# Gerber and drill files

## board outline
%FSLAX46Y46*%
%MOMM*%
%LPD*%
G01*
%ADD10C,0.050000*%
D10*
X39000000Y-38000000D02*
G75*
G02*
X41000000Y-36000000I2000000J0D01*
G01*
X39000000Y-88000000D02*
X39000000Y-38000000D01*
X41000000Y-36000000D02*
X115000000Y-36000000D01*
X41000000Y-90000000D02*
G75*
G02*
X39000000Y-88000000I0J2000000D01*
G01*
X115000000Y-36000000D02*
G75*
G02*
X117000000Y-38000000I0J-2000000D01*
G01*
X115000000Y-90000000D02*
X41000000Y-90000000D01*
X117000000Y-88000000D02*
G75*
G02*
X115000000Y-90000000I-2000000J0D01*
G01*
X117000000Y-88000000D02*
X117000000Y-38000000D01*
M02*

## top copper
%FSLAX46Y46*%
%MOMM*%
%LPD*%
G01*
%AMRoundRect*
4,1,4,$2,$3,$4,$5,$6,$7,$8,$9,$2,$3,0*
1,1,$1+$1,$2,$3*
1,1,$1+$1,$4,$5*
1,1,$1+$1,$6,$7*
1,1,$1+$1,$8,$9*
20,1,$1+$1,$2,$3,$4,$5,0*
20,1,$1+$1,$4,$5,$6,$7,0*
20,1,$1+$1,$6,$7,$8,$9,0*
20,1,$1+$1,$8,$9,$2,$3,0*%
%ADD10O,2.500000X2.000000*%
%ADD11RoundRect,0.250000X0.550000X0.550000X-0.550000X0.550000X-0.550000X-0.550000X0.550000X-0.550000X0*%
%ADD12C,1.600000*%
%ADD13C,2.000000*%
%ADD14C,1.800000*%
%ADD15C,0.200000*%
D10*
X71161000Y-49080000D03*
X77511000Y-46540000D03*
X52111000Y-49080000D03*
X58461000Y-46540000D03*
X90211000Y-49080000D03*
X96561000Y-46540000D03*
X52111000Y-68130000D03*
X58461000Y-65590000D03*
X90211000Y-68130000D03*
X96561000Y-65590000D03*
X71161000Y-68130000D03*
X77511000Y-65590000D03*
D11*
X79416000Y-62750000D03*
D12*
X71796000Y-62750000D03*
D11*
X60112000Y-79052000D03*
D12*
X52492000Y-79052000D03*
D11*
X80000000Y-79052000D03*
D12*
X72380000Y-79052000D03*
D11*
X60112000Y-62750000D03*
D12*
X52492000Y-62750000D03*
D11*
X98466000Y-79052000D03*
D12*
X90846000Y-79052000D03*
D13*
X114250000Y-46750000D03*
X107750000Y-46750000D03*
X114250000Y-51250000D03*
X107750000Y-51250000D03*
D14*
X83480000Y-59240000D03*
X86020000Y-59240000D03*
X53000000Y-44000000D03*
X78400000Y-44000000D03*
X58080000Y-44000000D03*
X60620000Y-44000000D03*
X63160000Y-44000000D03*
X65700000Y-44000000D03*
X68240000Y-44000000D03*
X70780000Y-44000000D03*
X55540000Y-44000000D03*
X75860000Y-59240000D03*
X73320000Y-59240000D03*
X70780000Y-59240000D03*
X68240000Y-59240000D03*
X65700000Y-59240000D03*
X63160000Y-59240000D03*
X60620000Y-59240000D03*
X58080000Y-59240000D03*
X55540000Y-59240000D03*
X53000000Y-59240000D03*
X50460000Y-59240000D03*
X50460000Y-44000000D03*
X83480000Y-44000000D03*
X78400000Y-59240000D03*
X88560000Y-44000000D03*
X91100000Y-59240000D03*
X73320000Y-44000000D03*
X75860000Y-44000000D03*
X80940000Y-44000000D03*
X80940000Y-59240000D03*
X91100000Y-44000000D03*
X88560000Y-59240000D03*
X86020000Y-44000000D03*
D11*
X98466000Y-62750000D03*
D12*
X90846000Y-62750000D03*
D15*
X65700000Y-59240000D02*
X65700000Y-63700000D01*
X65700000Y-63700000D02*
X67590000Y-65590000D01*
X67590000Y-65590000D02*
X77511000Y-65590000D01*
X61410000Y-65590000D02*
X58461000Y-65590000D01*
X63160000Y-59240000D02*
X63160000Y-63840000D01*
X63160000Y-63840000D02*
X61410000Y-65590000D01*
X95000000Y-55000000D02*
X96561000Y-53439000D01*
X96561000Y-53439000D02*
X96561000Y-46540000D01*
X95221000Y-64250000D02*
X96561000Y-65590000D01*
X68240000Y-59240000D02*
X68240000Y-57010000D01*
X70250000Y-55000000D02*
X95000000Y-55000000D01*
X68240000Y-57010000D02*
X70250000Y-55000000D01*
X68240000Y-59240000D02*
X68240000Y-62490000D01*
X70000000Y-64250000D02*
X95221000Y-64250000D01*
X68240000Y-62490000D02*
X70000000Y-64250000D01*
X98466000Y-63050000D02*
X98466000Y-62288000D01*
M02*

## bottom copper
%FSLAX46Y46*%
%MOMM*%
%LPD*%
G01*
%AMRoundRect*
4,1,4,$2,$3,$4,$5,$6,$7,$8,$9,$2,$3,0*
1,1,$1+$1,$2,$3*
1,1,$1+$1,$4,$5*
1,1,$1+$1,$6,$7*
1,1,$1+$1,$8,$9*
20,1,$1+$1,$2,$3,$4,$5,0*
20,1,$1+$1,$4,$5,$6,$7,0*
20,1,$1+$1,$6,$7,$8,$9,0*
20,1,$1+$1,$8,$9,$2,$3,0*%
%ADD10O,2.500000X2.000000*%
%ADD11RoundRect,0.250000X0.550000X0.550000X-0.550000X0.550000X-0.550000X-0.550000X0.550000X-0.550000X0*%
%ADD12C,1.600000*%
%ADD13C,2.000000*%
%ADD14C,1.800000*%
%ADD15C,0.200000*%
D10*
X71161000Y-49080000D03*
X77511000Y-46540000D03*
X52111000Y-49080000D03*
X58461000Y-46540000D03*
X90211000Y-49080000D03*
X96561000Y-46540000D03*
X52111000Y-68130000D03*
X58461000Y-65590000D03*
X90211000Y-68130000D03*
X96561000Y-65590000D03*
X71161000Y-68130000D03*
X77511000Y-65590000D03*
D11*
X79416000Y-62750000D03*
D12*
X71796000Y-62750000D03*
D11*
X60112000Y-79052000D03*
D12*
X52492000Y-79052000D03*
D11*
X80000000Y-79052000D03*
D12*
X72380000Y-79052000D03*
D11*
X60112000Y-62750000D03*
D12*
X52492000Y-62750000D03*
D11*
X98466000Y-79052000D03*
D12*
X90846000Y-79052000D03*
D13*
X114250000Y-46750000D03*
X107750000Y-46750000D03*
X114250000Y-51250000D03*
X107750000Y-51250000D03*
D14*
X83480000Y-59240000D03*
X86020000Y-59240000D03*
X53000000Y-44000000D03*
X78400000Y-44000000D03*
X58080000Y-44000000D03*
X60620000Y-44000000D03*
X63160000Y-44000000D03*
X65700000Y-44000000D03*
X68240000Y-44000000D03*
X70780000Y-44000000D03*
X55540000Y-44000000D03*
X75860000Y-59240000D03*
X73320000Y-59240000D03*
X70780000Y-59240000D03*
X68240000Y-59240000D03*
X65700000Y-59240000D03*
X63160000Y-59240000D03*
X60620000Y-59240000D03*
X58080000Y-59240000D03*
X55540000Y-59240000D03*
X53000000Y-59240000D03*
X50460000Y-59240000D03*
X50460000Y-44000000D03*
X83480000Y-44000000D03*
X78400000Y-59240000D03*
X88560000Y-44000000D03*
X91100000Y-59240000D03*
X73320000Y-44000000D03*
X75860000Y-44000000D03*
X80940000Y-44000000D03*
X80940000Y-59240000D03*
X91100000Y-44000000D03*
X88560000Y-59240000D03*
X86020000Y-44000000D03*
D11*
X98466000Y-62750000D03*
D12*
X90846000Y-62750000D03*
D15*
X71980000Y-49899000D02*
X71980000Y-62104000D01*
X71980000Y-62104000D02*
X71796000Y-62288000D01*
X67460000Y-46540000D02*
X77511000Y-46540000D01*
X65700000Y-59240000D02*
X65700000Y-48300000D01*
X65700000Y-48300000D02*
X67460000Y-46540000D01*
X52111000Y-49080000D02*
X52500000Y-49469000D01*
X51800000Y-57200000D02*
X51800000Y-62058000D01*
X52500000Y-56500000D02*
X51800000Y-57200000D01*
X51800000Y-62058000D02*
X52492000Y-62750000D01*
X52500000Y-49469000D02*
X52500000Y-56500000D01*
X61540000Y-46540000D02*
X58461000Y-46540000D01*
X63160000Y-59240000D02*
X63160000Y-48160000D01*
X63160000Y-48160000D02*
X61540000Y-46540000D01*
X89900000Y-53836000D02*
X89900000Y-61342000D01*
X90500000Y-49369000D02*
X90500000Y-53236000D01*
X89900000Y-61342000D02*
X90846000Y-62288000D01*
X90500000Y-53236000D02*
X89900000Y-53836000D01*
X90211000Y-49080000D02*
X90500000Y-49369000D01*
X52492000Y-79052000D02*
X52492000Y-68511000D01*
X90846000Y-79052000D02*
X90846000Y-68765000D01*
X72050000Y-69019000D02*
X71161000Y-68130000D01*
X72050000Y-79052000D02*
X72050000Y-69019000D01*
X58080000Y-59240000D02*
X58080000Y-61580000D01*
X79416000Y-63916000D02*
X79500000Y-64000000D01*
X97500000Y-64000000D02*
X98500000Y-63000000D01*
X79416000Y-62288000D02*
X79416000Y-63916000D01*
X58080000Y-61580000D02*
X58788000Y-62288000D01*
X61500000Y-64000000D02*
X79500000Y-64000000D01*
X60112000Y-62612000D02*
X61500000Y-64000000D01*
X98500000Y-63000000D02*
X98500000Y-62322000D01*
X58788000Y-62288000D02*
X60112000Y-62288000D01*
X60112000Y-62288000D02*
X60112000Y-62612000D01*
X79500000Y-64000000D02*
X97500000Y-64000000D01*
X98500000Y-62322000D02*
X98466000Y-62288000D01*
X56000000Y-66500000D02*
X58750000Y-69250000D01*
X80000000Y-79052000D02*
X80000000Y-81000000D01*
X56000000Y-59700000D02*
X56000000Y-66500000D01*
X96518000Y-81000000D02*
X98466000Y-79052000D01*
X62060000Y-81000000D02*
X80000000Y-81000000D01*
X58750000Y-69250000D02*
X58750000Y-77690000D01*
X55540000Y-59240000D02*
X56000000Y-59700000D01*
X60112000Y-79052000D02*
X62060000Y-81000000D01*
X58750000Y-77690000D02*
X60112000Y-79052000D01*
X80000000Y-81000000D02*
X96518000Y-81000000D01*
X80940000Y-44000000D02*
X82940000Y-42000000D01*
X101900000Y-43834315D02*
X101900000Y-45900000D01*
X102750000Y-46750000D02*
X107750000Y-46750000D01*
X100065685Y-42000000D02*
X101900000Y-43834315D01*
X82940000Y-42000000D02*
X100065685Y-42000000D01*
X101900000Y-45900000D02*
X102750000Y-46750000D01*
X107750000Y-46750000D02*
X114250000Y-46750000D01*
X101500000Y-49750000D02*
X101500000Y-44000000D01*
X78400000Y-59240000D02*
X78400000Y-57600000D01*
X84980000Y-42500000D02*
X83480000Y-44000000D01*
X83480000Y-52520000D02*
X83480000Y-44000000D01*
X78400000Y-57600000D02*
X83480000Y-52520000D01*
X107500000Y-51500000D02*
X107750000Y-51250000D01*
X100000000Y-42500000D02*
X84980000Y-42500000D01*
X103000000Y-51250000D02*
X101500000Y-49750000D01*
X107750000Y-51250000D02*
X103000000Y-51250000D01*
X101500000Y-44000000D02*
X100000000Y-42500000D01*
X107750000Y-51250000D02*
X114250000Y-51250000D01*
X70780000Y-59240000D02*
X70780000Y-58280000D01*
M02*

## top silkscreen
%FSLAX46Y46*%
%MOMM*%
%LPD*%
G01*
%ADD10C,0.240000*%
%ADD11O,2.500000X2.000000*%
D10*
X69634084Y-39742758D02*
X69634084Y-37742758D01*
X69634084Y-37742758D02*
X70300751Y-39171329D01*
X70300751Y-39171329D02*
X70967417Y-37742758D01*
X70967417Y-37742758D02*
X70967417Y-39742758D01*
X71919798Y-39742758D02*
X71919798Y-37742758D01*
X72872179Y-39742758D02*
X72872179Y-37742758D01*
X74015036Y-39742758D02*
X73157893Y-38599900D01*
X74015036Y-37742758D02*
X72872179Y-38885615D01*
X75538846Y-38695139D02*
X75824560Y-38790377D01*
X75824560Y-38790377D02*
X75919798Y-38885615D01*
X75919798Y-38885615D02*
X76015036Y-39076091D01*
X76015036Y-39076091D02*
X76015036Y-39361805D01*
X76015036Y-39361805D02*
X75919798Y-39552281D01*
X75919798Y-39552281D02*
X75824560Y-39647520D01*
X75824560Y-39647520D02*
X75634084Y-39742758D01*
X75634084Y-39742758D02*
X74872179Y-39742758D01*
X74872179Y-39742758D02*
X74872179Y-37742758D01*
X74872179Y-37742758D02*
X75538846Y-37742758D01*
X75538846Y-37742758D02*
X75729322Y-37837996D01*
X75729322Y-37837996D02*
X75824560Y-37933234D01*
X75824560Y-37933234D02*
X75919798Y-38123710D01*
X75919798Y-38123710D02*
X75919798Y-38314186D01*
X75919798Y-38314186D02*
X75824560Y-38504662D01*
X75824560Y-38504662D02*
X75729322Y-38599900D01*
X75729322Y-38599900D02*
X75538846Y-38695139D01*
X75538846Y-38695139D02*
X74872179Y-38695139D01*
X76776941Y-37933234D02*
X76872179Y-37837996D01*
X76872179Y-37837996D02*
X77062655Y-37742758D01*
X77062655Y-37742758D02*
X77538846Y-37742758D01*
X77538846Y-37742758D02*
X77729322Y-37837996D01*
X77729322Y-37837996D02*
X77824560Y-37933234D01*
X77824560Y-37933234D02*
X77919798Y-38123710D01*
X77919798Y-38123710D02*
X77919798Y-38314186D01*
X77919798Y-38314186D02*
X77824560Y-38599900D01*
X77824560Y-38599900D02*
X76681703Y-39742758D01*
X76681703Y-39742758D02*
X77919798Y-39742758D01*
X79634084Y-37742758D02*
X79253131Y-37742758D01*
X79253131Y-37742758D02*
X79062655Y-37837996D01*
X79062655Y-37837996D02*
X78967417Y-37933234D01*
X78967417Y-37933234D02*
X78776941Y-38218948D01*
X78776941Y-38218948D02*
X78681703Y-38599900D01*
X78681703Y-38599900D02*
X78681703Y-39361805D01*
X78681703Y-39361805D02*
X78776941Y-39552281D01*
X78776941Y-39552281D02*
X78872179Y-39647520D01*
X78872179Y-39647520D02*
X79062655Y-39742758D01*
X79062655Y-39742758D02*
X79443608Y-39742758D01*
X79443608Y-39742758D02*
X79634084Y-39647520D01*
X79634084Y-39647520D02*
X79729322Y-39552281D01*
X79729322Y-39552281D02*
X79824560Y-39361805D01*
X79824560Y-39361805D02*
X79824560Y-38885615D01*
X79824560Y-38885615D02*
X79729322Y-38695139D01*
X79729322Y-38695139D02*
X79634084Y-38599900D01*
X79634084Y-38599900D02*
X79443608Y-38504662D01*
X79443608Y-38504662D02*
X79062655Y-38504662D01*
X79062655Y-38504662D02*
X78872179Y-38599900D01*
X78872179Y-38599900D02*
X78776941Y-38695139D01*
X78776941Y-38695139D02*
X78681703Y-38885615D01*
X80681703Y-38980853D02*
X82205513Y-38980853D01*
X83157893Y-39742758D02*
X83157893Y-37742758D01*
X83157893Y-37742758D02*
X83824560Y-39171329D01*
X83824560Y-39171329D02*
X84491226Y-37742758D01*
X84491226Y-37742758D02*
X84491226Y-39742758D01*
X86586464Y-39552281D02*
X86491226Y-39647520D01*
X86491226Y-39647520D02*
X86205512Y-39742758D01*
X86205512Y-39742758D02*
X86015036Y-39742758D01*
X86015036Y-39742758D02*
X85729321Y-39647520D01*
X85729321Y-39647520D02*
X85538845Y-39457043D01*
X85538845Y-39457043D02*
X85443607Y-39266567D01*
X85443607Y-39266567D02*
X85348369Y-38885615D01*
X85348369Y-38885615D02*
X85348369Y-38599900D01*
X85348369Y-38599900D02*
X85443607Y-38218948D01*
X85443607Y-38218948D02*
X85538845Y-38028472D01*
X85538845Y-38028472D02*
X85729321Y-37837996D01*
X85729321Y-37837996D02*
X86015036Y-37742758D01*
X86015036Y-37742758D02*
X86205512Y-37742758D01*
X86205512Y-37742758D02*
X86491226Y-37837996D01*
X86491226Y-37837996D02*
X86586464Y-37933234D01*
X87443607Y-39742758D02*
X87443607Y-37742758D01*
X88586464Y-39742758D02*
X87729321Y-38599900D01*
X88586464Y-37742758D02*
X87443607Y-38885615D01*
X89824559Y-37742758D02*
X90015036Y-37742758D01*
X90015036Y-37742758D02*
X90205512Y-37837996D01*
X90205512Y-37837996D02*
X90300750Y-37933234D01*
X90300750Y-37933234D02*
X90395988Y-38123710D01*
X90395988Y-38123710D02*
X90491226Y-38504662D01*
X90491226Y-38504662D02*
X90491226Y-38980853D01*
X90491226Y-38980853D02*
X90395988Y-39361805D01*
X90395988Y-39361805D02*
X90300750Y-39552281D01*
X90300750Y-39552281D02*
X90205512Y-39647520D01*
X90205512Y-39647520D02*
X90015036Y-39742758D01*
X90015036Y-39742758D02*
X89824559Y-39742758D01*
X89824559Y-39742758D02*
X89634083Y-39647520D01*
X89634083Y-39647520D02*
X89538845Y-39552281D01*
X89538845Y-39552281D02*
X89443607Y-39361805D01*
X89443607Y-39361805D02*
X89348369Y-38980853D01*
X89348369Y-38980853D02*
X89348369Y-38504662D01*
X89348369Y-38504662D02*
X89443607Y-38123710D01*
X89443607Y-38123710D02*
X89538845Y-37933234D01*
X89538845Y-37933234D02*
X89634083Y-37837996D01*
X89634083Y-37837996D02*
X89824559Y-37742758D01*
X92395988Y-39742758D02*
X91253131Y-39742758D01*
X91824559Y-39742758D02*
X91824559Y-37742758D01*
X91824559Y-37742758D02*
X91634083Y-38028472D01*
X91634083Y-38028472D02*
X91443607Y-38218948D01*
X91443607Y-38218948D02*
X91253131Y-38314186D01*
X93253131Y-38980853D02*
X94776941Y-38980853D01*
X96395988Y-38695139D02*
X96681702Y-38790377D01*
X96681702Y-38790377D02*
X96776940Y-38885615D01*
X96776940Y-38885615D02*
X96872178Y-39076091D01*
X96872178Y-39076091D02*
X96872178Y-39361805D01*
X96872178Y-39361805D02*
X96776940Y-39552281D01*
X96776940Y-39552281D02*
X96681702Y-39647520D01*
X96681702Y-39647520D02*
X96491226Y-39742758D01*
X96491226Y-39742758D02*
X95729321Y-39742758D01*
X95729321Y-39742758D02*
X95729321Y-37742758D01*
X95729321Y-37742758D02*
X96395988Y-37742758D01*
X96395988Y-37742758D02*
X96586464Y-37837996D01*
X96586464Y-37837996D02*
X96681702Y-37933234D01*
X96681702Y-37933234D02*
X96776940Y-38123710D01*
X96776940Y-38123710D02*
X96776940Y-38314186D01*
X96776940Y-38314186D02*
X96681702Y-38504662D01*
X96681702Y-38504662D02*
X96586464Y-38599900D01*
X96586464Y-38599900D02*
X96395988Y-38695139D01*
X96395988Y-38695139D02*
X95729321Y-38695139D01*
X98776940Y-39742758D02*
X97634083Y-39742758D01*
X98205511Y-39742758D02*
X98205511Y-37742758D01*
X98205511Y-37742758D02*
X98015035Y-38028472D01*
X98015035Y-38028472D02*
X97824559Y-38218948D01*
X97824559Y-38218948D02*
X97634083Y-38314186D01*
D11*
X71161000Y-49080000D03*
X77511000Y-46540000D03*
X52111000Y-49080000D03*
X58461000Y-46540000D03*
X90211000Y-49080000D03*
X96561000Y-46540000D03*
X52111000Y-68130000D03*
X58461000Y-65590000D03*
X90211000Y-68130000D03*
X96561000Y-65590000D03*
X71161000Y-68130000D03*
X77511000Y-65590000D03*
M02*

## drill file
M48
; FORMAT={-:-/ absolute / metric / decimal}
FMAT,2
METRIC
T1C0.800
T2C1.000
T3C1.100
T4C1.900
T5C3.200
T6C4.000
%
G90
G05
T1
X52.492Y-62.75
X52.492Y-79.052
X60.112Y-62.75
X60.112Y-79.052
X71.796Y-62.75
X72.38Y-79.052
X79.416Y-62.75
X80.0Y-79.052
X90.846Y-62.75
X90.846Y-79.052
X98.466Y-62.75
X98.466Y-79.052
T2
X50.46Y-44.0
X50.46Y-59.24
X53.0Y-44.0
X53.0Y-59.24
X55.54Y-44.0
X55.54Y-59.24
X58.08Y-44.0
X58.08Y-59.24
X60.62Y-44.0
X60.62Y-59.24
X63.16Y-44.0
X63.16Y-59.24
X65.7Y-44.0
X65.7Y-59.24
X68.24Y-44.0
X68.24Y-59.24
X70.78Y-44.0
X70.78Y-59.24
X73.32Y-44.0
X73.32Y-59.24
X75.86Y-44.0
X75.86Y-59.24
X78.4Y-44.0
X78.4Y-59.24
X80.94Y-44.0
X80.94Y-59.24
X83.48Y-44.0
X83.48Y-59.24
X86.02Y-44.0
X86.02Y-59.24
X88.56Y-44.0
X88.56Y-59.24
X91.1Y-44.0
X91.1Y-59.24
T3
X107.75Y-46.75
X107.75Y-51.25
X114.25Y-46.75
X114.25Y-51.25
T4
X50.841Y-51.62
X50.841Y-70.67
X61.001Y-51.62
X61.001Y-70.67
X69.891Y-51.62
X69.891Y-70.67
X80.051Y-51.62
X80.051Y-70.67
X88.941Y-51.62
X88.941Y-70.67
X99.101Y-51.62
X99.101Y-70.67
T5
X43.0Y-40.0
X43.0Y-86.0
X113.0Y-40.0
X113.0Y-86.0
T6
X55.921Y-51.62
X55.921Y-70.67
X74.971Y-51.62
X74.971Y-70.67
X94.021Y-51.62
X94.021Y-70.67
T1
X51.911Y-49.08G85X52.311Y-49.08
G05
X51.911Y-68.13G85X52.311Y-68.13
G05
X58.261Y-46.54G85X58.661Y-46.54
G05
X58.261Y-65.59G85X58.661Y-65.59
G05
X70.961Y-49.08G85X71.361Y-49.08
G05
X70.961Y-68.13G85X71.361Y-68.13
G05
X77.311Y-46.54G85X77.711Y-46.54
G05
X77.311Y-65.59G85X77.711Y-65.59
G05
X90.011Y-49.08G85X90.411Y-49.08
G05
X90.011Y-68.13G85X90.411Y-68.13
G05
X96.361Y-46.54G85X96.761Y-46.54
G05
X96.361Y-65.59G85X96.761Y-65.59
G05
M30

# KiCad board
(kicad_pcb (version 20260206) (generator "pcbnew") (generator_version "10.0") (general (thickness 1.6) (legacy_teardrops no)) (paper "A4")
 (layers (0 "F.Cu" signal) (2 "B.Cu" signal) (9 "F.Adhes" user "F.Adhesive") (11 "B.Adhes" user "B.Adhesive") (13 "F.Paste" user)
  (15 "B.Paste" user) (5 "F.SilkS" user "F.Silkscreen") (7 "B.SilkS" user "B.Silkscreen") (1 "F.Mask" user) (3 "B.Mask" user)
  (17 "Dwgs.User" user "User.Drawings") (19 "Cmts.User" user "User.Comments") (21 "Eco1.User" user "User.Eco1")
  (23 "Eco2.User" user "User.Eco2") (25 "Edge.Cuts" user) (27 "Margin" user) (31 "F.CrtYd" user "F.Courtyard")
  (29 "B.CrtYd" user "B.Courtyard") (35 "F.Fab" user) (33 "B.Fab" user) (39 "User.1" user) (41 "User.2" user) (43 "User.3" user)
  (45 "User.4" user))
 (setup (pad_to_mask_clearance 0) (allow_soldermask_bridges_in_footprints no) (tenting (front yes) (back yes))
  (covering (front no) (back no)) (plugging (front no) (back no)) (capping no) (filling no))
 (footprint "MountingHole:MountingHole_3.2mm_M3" (layer "F.Cu") (at 113 40 180)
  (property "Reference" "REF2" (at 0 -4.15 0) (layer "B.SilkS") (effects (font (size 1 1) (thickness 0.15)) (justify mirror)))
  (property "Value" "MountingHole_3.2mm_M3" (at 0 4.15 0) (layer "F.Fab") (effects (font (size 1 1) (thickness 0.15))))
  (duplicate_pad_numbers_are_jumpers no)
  (pad "" np_thru_hole circle (at 0 0 180) (size 3.2 3.2) (drill 3.2) (layers "*.Cu" "*.Mask")))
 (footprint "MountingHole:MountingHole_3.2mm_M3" (layer "F.Cu") (at 113 86)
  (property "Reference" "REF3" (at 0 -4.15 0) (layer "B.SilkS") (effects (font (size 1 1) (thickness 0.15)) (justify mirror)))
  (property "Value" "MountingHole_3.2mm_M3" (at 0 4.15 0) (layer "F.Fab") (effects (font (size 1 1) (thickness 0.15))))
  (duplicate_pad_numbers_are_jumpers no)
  (pad "" np_thru_hole circle (at 0 0) (size 3.2 3.2) (drill 3.2) (layers "*.Cu" "*.Mask")))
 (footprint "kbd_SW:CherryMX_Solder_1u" (layer "F.Cu") (at 74.971 51.62)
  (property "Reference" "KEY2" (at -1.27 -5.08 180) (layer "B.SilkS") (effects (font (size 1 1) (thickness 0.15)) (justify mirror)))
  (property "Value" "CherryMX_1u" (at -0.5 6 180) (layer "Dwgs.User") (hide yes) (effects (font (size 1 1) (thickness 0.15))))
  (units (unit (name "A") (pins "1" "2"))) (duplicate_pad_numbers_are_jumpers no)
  (pad "" np_thru_hole circle (at -5.08 0 90) (size 1.9 1.9) (drill 1.9) (layers "*.Cu" "*.Mask"))
  (pad "" np_thru_hole circle (at 0 0 90) (size 4 4) (drill 4) (layers "*.Cu" "*.Mask"))
  (pad "" np_thru_hole circle (at 5.08 0 90) (size 1.9 1.9) (drill 1.9) (layers "*.Cu" "*.Mask"))
  (pad "1" thru_hole oval (at -3.81 -2.54) (size 2.5 2) (drill oval 1.2 0.8) (layers "*.Cu" "B.Mask" "F.SilkS") (remove_unused_layers no)
   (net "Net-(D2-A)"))
  (pad "2" thru_hole oval (at 2.54 -5.08) (size 2.5 2) (drill oval 1.2 0.8) (layers "*.Cu" "B.Mask" "F.SilkS") (remove_unused_layers no)
   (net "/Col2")))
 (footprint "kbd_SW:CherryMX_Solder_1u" (layer "F.Cu") (at 55.921 51.62)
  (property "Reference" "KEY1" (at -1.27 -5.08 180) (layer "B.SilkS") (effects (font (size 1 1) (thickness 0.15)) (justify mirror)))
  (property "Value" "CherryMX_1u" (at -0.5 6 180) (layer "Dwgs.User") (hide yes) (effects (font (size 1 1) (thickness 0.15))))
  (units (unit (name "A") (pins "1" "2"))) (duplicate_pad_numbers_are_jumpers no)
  (pad "" np_thru_hole circle (at -5.08 0 90) (size 1.9 1.9) (drill 1.9) (layers "*.Cu" "*.Mask"))
  (pad "" np_thru_hole circle (at 0 0 90) (size 4 4) (drill 4) (layers "*.Cu" "*.Mask"))
  (pad "" np_thru_hole circle (at 5.08 0 90) (size 1.9 1.9) (drill 1.9) (layers "*.Cu" "*.Mask"))
  (pad "1" thru_hole oval (at -3.81 -2.54) (size 2.5 2) (drill oval 1.2 0.8) (layers "*.Cu" "B.Mask" "F.SilkS") (remove_unused_layers no)
   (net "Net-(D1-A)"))
  (pad "2" thru_hole oval (at 2.54 -5.08) (size 2.5 2) (drill oval 1.2 0.8) (layers "*.Cu" "B.Mask" "F.SilkS") (remove_unused_layers no)
   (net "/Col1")))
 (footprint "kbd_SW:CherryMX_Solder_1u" (layer "F.Cu") (at 94.021 51.62)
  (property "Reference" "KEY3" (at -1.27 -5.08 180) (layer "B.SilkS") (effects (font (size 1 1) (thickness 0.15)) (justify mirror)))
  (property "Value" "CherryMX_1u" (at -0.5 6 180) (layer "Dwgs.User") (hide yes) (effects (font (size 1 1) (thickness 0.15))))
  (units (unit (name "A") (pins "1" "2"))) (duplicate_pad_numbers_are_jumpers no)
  (pad "" np_thru_hole circle (at -5.08 0 90) (size 1.9 1.9) (drill 1.9) (layers "*.Cu" "*.Mask"))
  (pad "" np_thru_hole circle (at 0 0 90) (size 4 4) (drill 4) (layers "*.Cu" "*.Mask"))
  (pad "" np_thru_hole circle (at 5.08 0 90) (size 1.9 1.9) (drill 1.9) (layers "*.Cu" "*.Mask"))
  (pad "1" thru_hole oval (at -3.81 -2.54) (size 2.5 2) (drill oval 1.2 0.8) (layers "*.Cu" "B.Mask" "F.SilkS") (remove_unused_layers no)
   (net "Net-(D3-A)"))
  (pad "2" thru_hole oval (at 2.54 -5.08) (size 2.5 2) (drill oval 1.2 0.8) (layers "*.Cu" "B.Mask" "F.SilkS") (remove_unused_layers no)
   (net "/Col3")))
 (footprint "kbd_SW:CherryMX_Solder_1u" (layer "F.Cu") (at 55.921 70.67)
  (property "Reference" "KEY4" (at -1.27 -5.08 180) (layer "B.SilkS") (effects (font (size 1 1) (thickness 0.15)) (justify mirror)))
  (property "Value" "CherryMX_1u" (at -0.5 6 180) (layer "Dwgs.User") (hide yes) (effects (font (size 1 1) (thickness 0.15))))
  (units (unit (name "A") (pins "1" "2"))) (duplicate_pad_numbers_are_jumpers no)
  (pad "" np_thru_hole circle (at -5.08 0 90) (size 1.9 1.9) (drill 1.9) (layers "*.Cu" "*.Mask"))
  (pad "" np_thru_hole circle (at 0 0 90) (size 4 4) (drill 4) (layers "*.Cu" "*.Mask"))
  (pad "" np_thru_hole circle (at 5.08 0 90) (size 1.9 1.9) (drill 1.9) (layers "*.Cu" "*.Mask"))
  (pad "1" thru_hole oval (at -3.81 -2.54) (size 2.5 2) (drill oval 1.2 0.8) (layers "*.Cu" "B.Mask" "F.SilkS") (remove_unused_layers no)
   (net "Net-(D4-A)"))
  (pad "2" thru_hole oval (at 2.54 -5.08) (size 2.5 2) (drill oval 1.2 0.8) (layers "*.Cu" "B.Mask" "F.SilkS") (remove_unused_layers no)
   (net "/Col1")))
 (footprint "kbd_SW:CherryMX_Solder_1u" (layer "F.Cu") (at 94.021 70.67)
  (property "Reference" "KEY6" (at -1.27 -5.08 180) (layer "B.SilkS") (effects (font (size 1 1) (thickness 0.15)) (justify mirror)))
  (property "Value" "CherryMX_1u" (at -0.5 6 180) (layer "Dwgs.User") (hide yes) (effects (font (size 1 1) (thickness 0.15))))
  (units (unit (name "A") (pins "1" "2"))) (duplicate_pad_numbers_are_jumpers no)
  (pad "" np_thru_hole circle (at -5.08 0 90) (size 1.9 1.9) (drill 1.9) (layers "*.Cu" "*.Mask"))
  (pad "" np_thru_hole circle (at 0 0 90) (size 4 4) (drill 4) (layers "*.Cu" "*.Mask"))
  (pad "" np_thru_hole circle (at 5.08 0 90) (size 1.9 1.9) (drill 1.9) (layers "*.Cu" "*.Mask"))
  (pad "1" thru_hole oval (at -3.81 -2.54) (size 2.5 2) (drill oval 1.2 0.8) (layers "*.Cu" "B.Mask" "F.SilkS") (remove_unused_layers no)
   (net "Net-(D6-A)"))
  (pad "2" thru_hole oval (at 2.54 -5.08) (size 2.5 2) (drill oval 1.2 0.8) (layers "*.Cu" "B.Mask" "F.SilkS") (remove_unused_layers no)
   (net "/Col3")))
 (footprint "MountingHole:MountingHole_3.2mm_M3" (layer "F.Cu") (at 43 40 180)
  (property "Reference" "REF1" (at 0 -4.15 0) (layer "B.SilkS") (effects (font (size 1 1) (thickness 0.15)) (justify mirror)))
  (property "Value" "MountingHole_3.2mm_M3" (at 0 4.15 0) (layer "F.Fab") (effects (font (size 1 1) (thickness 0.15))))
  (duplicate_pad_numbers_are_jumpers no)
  (pad "" np_thru_hole circle (at 0 0 180) (size 3.2 3.2) (drill 3.2) (layers "*.Cu" "*.Mask")))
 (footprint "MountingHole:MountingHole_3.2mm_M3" (layer "F.Cu") (at 43 86)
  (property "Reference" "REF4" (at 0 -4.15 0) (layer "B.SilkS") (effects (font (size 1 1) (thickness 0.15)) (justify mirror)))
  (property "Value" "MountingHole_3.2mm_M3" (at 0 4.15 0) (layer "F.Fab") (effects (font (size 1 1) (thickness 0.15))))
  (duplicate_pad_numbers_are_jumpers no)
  (pad "" np_thru_hole circle (at 0 0) (size 3.2 3.2) (drill 3.2) (layers "*.Cu" "*.Mask")))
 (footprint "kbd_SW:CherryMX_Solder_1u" (layer "F.Cu") (at 74.971 70.67)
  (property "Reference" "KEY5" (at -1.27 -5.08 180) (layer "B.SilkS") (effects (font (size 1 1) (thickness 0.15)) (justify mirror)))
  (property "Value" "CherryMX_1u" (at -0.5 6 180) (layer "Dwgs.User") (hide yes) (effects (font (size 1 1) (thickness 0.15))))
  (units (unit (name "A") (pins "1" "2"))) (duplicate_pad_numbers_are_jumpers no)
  (pad "" np_thru_hole circle (at -5.08 0 90) (size 1.9 1.9) (drill 1.9) (layers "*.Cu" "*.Mask"))
  (pad "" np_thru_hole circle (at 0 0 90) (size 4 4) (drill 4) (layers "*.Cu" "*.Mask"))
  (pad "" np_thru_hole circle (at 5.08 0 90) (size 1.9 1.9) (drill 1.9) (layers "*.Cu" "*.Mask"))
  (pad "1" thru_hole oval (at -3.81 -2.54) (size 2.5 2) (drill oval 1.2 0.8) (layers "*.Cu" "B.Mask" "F.SilkS") (remove_unused_layers no)
   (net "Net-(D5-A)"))
  (pad "2" thru_hole oval (at 2.54 -5.08) (size 2.5 2) (drill oval 1.2 0.8) (layers "*.Cu" "B.Mask" "F.SilkS") (remove_unused_layers no)
   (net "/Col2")))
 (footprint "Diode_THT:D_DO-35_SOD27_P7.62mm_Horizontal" (layer "B.Cu") (at 79.416 62.75 180)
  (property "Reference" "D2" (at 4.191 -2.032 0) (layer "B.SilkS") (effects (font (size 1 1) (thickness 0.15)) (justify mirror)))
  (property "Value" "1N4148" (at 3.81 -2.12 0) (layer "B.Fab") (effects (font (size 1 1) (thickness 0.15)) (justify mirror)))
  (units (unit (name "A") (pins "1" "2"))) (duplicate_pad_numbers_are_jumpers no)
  (pad "1" thru_hole roundrect (at 0 0 180) (size 1.6 1.6) (drill 0.8) (layers "*.Cu" "*.Mask") (remove_unused_layers no)
   (roundrect_rratio 0.15625) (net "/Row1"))
  (pad "2" thru_hole circle (at 7.62 0 180) (size 1.6 1.6) (drill 0.8) (layers "*.Cu" "*.Mask") (remove_unused_layers no) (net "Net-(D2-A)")))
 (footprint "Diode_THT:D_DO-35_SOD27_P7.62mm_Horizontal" (layer "B.Cu") (at 60.112 79.052 180)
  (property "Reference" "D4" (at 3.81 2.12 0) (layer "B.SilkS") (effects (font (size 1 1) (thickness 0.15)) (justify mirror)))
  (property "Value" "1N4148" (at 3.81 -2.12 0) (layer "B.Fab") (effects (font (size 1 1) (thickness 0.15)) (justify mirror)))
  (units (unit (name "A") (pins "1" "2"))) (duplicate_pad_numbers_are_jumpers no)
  (pad "1" thru_hole roundrect (at 0 0 180) (size 1.6 1.6) (drill 0.8) (layers "*.Cu" "*.Mask") (remove_unused_layers no)
   (roundrect_rratio 0.15625) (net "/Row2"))
  (pad "2" thru_hole circle (at 7.62 0 180) (size 1.6 1.6) (drill 0.8) (layers "*.Cu" "*.Mask") (remove_unused_layers no) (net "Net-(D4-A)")))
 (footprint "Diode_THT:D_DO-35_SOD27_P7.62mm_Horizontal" (layer "B.Cu") (at 80 79.052 180)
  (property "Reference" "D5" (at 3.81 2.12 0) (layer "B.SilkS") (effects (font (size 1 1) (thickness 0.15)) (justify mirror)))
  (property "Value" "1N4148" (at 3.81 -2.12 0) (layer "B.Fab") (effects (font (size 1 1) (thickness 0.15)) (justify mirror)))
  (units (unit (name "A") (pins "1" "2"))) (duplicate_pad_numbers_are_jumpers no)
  (pad "1" thru_hole roundrect (at 0 0 180) (size 1.6 1.6) (drill 0.8) (layers "*.Cu" "*.Mask") (remove_unused_layers no)
   (roundrect_rratio 0.15625) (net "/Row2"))
  (pad "2" thru_hole circle (at 7.62 0 180) (size 1.6 1.6) (drill 0.8) (layers "*.Cu" "*.Mask") (remove_unused_layers no) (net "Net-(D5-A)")))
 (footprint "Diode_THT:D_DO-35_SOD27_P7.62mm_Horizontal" (layer "B.Cu") (at 60.112 62.75 180)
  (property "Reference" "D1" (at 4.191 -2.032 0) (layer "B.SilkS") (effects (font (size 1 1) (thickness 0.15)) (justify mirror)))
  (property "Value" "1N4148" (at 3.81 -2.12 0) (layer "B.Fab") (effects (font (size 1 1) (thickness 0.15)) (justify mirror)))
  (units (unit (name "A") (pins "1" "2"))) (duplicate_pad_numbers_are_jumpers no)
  (pad "1" thru_hole roundrect (at 0 0 180) (size 1.6 1.6) (drill 0.8) (layers "*.Cu" "*.Mask") (remove_unused_layers no)
   (roundrect_rratio 0.15625) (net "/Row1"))
  (pad "2" thru_hole circle (at 7.62 0 180) (size 1.6 1.6) (drill 0.8) (layers "*.Cu" "*.Mask") (remove_unused_layers no) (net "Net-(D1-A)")))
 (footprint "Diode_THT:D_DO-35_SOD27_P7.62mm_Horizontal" (layer "B.Cu") (at 98.466 79.052 180)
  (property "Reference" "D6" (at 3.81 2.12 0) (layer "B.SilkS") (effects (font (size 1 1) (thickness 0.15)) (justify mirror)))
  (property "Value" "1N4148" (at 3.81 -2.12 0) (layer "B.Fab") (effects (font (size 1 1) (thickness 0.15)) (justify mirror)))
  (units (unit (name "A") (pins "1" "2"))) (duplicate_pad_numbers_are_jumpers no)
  (pad "1" thru_hole roundrect (at 0 0 180) (size 1.6 1.6) (drill 0.8) (layers "*.Cu" "*.Mask") (remove_unused_layers no)
   (roundrect_rratio 0.15625) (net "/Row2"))
  (pad "2" thru_hole circle (at 7.62 0 180) (size 1.6 1.6) (drill 0.8) (layers "*.Cu" "*.Mask") (remove_unused_layers no) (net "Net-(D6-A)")))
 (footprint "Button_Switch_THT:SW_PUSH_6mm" (layer "B.Cu") (at 114.25 46.75 180)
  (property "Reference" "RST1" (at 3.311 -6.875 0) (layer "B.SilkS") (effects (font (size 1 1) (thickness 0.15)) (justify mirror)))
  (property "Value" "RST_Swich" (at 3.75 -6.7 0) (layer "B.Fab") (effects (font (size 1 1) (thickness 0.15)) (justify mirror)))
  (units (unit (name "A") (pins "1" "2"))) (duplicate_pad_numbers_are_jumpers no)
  (pad "1" thru_hole circle (at 0 0 90) (size 2 2) (drill 1.1) (layers "*.Cu" "*.Mask") (remove_unused_layers no) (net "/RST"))
  (pad "1" thru_hole circle (at 6.5 0 90) (size 2 2) (drill 1.1) (layers "*.Cu" "*.Mask") (remove_unused_layers no) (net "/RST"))
  (pad "2" thru_hole circle (at 0 -4.5 90) (size 2 2) (drill 1.1) (layers "*.Cu" "*.Mask") (remove_unused_layers no) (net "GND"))
  (pad "2" thru_hole circle (at 6.5 -4.5 90) (size 2 2) (drill 1.1) (layers "*.Cu" "*.Mask") (remove_unused_layers no) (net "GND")))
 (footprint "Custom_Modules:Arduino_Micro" (layer "B.Cu") (at 50.46 51.62 -90)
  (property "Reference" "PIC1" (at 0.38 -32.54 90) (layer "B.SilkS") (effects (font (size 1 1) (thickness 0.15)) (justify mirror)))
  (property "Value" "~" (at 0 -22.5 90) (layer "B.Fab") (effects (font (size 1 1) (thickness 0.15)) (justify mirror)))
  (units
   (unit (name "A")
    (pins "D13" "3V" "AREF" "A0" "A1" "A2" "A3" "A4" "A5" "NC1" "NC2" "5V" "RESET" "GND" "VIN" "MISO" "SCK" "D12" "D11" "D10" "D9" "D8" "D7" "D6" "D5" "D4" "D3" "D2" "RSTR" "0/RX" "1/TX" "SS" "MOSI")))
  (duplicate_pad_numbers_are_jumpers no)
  (pad "0/RX" thru_hole circle (at 7.62 -33.02 270) (size 1.8 1.8) (drill 1) (layers "*.Cu" "*.Mask") (remove_unused_layers no)
   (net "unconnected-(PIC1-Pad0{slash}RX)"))
  (pad "1/TX" thru_hole circle (at 7.62 -35.56 270) (size 1.8 1.8) (drill 1) (layers "*.Cu" "*.Mask") (remove_unused_layers no)
   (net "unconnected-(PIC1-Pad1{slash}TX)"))
  (pad "3V" thru_hole circle (at -7.62 -2.54 270) (size 1.8 1.8) (drill 1) (layers "*.Cu" "*.Mask") (remove_unused_layers no)
   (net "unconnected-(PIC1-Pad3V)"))
  (pad "5V" thru_hole circle (at -7.62 -27.94 270) (size 1.8 1.8) (drill 1) (layers "*.Cu" "*.Mask") (remove_unused_layers no)
   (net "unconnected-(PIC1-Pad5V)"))
  (pad "A0" thru_hole circle (at -7.62 -7.62 270) (size 1.8 1.8) (drill 1) (layers "*.Cu" "*.Mask") (remove_unused_layers no)
   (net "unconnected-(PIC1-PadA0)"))
  (pad "A1" thru_hole circle (at -7.62 -10.16 270) (size 1.8 1.8) (drill 1) (layers "*.Cu" "*.Mask") (remove_unused_layers no)
   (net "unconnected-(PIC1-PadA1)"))
  (pad "A2" thru_hole circle (at -7.62 -12.7 270) (size 1.8 1.8) (drill 1) (layers "*.Cu" "*.Mask") (remove_unused_layers no)
   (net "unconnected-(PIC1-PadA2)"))
  (pad "A3" thru_hole circle (at -7.62 -15.24 270) (size 1.8 1.8) (drill 1) (layers "*.Cu" "*.Mask") (remove_unused_layers no)
   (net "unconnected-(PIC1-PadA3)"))
  (pad "A4" thru_hole circle (at -7.62 -17.78 270) (size 1.8 1.8) (drill 1) (layers "*.Cu" "*.Mask") (remove_unused_layers no)
   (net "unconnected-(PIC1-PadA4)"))
  (pad "A5" thru_hole circle (at -7.62 -20.32 270) (size 1.8 1.8) (drill 1) (layers "*.Cu" "*.Mask") (remove_unused_layers no)
   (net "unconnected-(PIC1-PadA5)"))
  (pad "AREF" thru_hole circle (at -7.62 -5.08 270) (size 1.8 1.8) (drill 1) (layers "*.Cu" "*.Mask") (remove_unused_layers no)
   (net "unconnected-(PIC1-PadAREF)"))
  (pad "D2" thru_hole circle (at 7.62 -25.4 270) (size 1.8 1.8) (drill 1) (layers "*.Cu" "*.Mask") (remove_unused_layers no)
   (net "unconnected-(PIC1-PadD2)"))
  (pad "D3" thru_hole circle (at 7.62 -22.86 270) (size 1.8 1.8) (drill 1) (layers "*.Cu" "*.Mask") (remove_unused_layers no)
   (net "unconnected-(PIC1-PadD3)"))
  (pad "D4" thru_hole circle (at 7.62 -20.32 270) (size 1.8 1.8) (drill 1) (layers "*.Cu" "*.Mask") (remove_unused_layers no)
   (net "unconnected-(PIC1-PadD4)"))
  (pad "D5" thru_hole circle (at 7.62 -17.78 270) (size 1.8 1.8) (drill 1) (layers "*.Cu" "*.Mask") (remove_unused_layers no) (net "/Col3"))
  (pad "D6" thru_hole circle (at 7.62 -15.24 270) (size 1.8 1.8) (drill 1) (layers "*.Cu" "*.Mask") (remove_unused_layers no) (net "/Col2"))
  (pad "D7" thru_hole circle (at 7.62 -12.7 270) (size 1.8 1.8) (drill 1) (layers "*.Cu" "*.Mask") (remove_unused_layers no) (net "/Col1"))
  (pad "D8" thru_hole circle (at 7.62 -10.16 270) (size 1.8 1.8) (drill 1) (layers "*.Cu" "*.Mask") (remove_unused_layers no)
   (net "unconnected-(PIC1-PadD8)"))
  (pad "D9" thru_hole circle (at 7.62 -7.62 270) (size 1.8 1.8) (drill 1) (layers "*.Cu" "*.Mask") (remove_unused_layers no) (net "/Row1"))
  (pad "D10" thru_hole circle (at 7.62 -5.08 270) (size 1.8 1.8) (drill 1) (layers "*.Cu" "*.Mask") (remove_unused_layers no) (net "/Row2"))
  (pad "D11" thru_hole circle (at 7.62 -2.54 270) (size 1.8 1.8) (drill 1) (layers "*.Cu" "*.Mask") (remove_unused_layers no)
   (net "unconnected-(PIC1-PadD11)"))
  (pad "D12" thru_hole circle (at 7.62 0 270) (size 1.8 1.8) (drill 1) (layers "*.Cu" "*.Mask") (remove_unused_layers no)
   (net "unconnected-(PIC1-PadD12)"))
  (pad "D13" thru_hole circle (at -7.62 0 270) (size 1.8 1.8) (drill 1) (layers "*.Cu" "*.Mask") (remove_unused_layers no)
   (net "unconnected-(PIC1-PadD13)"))
  (pad "GND" thru_hole circle (at -7.62 -33.02 270) (size 1.8 1.8) (drill 1) (layers "*.Cu" "*.Mask") (remove_unused_layers no) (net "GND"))
  (pad "GND" thru_hole circle (at 7.62 -27.94 270) (size 1.8 1.8) (drill 1) (layers "*.Cu" "*.Mask") (remove_unused_layers no) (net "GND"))
  (pad "MISO" thru_hole circle (at -7.62 -38.1 270) (size 1.8 1.8) (drill 1) (layers "*.Cu" "*.Mask") (remove_unused_layers no)
   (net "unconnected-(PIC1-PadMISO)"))
  (pad "MOSI" thru_hole circle (at 7.62 -40.64 270) (size 1.8 1.8) (drill 1) (layers "*.Cu" "*.Mask") (remove_unused_layers no)
   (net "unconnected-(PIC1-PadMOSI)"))
  (pad "NC1" thru_hole circle (at -7.62 -22.86 270) (size 1.8 1.8) (drill 1) (layers "*.Cu" "*.Mask") (remove_unused_layers no)
   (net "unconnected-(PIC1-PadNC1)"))
  (pad "NC2" thru_hole circle (at -7.62 -25.4 270) (size 1.8 1.8) (drill 1) (layers "*.Cu" "*.Mask") (remove_unused_layers no)
   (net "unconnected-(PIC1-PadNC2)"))
  (pad "RESET" thru_hole circle (at -7.62 -30.48 270) (size 1.8 1.8) (drill 1) (layers "*.Cu" "*.Mask") (remove_unused_layers no)
   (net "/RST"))
  (pad "RSTR" thru_hole circle (at 7.62 -30.48 270) (size 1.8 1.8) (drill 1) (layers "*.Cu" "*.Mask") (remove_unused_layers no)
   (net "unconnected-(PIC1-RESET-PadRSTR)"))
  (pad "SCK" thru_hole circle (at -7.62 -40.64 270) (size 1.8 1.8) (drill 1) (layers "*.Cu" "*.Mask") (remove_unused_layers no)
   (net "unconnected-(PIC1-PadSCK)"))
  (pad "SS" thru_hole circle (at 7.62 -38.1 270) (size 1.8 1.8) (drill 1) (layers "*.Cu" "*.Mask") (remove_unused_layers no)
   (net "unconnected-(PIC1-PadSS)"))
  (pad "VIN" thru_hole circle (at -7.62 -35.56 270) (size 1.8 1.8) (drill 1) (layers "*.Cu" "*.Mask") (remove_unused_layers no)
   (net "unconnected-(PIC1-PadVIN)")))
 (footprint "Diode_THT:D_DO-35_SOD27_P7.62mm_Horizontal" (layer "B.Cu") (at 98.466 62.75 180)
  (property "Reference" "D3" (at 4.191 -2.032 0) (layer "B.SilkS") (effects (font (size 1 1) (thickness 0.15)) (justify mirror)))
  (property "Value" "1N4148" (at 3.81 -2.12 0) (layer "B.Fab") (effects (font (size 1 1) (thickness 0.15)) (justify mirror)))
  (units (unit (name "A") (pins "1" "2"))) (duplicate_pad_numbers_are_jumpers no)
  (pad "1" thru_hole roundrect (at 0 0 180) (size 1.6 1.6) (drill 0.8) (layers "*.Cu" "*.Mask") (remove_unused_layers no)
   (roundrect_rratio 0.15625) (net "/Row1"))
  (pad "2" thru_hole circle (at 7.62 0 180) (size 1.6 1.6) (drill 0.8) (layers "*.Cu" "*.Mask") (remove_unused_layers no) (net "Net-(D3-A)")))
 (gr_arc (start 39 38) (mid 39.585786 36.585786) (end 41 36) (stroke (width 0.05) (type default)) (layer "Edge.Cuts"))
 (gr_line (start 39 88) (end 39 38) (stroke (width 0.05) (type default)) (layer "Edge.Cuts"))
 (gr_line (start 41 36) (end 115 36) (stroke (width 0.05) (type default)) (layer "Edge.Cuts"))
 (gr_arc (start 41 90) (mid 39.585786 89.414214) (end 39 88) (stroke (width 0.05) (type default)) (layer "Edge.Cuts"))
 (gr_arc (start 115 36) (mid 116.414214 36.585786) (end 117 38) (stroke (width 0.05) (type default)) (layer "Edge.Cuts"))
 (gr_line (start 115 90) (end 41 90) (stroke (width 0.05) (type default)) (layer "Edge.Cuts"))
 (gr_arc (start 117 88) (mid 116.414214 89.414214) (end 115 90) (stroke (width 0.05) (type default)) (layer "Edge.Cuts"))
 (gr_line (start 117 88) (end 117 38) (stroke (width 0.05) (type default)) (layer "Edge.Cuts"))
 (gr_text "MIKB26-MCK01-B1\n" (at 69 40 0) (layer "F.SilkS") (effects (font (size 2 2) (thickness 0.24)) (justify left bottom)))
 (segment (start 71.98 49.899) (end 71.98 62.104) (width 0.2) (layer "B.Cu") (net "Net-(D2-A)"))
 (segment (start 71.98 62.104) (end 71.796 62.288) (width 0.2) (layer "B.Cu") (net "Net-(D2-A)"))
 (segment (start 65.7 59.24) (end 65.7 63.7) (width 0.2) (layer "F.Cu") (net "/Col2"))
 (segment (start 65.7 63.7) (end 67.59 65.59) (width 0.2) (layer "F.Cu") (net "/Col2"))
 (segment (start 67.59 65.59) (end 77.511 65.59) (width 0.2) (layer "F.Cu") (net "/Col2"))
 (segment (start 67.46 46.54) (end 77.511 46.54) (width 0.2) (layer "B.Cu") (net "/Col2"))
 (segment (start 65.7 59.24) (end 65.7 48.3) (width 0.2) (layer "B.Cu") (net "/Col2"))
 (segment (start 65.7 48.3) (end 67.46 46.54) (width 0.2) (layer "B.Cu") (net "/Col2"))
 (segment (start 52.111 49.08) (end 52.5 49.469) (width 0.2) (layer "B.Cu") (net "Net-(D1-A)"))
 (segment (start 51.8 57.2) (end 51.8 62.058) (width 0.2) (layer "B.Cu") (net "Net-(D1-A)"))
 (segment (start 52.5 56.5) (end 51.8 57.2) (width 0.2) (layer "B.Cu") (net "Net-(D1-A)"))
 (segment (start 51.8 62.058) (end 52.492 62.75) (width 0.2) (layer "B.Cu") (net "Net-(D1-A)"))
 (segment (start 52.5 49.469) (end 52.5 56.5) (width 0.2) (layer "B.Cu") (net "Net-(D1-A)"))
 (segment (start 61.41 65.59) (end 58.461 65.59) (width 0.2) (layer "F.Cu") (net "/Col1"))
 (segment (start 63.16 59.24) (end 63.16 63.84) (width 0.2) (layer "F.Cu") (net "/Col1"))
 (segment (start 63.16 63.84) (end 61.41 65.59) (width 0.2) (layer "F.Cu") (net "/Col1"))
 (segment (start 61.54 46.54) (end 58.461 46.54) (width 0.2) (layer "B.Cu") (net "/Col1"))
 (segment (start 63.16 59.24) (end 63.16 48.16) (width 0.2) (layer "B.Cu") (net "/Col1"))
 (segment (start 63.16 48.16) (end 61.54 46.54) (width 0.2) (layer "B.Cu") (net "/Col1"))
 (segment (start 89.9 53.836) (end 89.9 61.342) (width 0.2) (layer "B.Cu") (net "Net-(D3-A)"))
 (segment (start 90.5 49.369) (end 90.5 53.236) (width 0.2) (layer "B.Cu") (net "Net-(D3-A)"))
 (segment (start 89.9 61.342) (end 90.846 62.288) (width 0.2) (layer "B.Cu") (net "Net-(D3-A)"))
 (segment (start 90.5 53.236) (end 89.9 53.836) (width 0.2) (layer "B.Cu") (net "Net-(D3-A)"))
 (segment (start 90.211 49.08) (end 90.5 49.369) (width 0.2) (layer "B.Cu") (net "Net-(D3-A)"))
 (segment (start 95 55) (end 96.561 53.439) (width 0.2) (layer "F.Cu") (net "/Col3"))
 (segment (start 96.561 53.439) (end 96.561 46.54) (width 0.2) (layer "F.Cu") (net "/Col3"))
 (segment (start 95.221 64.25) (end 96.561 65.59) (width 0.2) (layer "F.Cu") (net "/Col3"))
 (segment (start 68.24 59.24) (end 68.24 57.01) (width 0.2) (layer "F.Cu") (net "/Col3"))
 (segment (start 70.25 55) (end 95 55) (width 0.2) (layer "F.Cu") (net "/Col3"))
 (segment (start 68.24 57.01) (end 70.25 55) (width 0.2) (layer "F.Cu") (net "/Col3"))
 (segment (start 68.24 59.24) (end 68.24 62.49) (width 0.2) (layer "F.Cu") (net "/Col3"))
 (segment (start 70 64.25) (end 95.221 64.25) (width 0.2) (layer "F.Cu") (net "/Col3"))
 (segment (start 68.24 62.49) (end 70 64.25) (width 0.2) (layer "F.Cu") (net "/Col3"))
 (segment (start 52.492 79.052) (end 52.492 68.511) (width 0.2) (layer "B.Cu") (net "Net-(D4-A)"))
 (segment (start 90.846 79.052) (end 90.846 68.765) (width 0.2) (layer "B.Cu") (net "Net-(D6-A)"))
 (segment (start 72.05 69.019) (end 71.161 68.13) (width 0.2) (layer "B.Cu") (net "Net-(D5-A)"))
 (segment (start 72.05 79.052) (end 72.05 69.019) (width 0.2) (layer "B.Cu") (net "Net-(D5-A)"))
 (segment (start 98.466 63.05) (end 98.466 62.288) (width 0.2) (layer "F.Cu") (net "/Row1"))
 (segment (start 58.08 59.24) (end 58.08 61.58) (width 0.2) (layer "B.Cu") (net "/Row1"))
 (segment (start 79.416 63.916) (end 79.5 64) (width 0.2) (layer "B.Cu") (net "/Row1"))
 (segment (start 97.5 64) (end 98.5 63) (width 0.2) (layer "B.Cu") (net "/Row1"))
 (segment (start 79.416 62.288) (end 79.416 63.916) (width 0.2) (layer "B.Cu") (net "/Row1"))
 (segment (start 58.08 61.58) (end 58.788 62.288) (width 0.2) (layer "B.Cu") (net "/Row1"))
 (segment (start 61.5 64) (end 79.5 64) (width 0.2) (layer "B.Cu") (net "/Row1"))
 (segment (start 60.112 62.612) (end 61.5 64) (width 0.2) (layer "B.Cu") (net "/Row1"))
 (segment (start 98.5 63) (end 98.5 62.322) (width 0.2) (layer "B.Cu") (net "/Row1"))
 (segment (start 58.788 62.288) (end 60.112 62.288) (width 0.2) (layer "B.Cu") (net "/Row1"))
 (segment (start 60.112 62.288) (end 60.112 62.612) (width 0.2) (layer "B.Cu") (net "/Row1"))
 (segment (start 79.5 64) (end 97.5 64) (width 0.2) (layer "B.Cu") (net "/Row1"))
 (segment (start 98.5 62.322) (end 98.466 62.288) (width 0.2) (layer "B.Cu") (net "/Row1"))
 (segment (start 56 66.5) (end 58.75 69.25) (width 0.2) (layer "B.Cu") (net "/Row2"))
 (segment (start 80 79.052) (end 80 81) (width 0.2) (layer "B.Cu") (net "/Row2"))
 (segment (start 56 59.7) (end 56 66.5) (width 0.2) (layer "B.Cu") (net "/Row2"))
 (segment (start 96.518 81) (end 98.466 79.052) (width 0.2) (layer "B.Cu") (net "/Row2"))
 (segment (start 62.06 81) (end 80 81) (width 0.2) (layer "B.Cu") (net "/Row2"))
 (segment (start 58.75 69.25) (end 58.75 77.69) (width 0.2) (layer "B.Cu") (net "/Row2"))
 (segment (start 55.54 59.24) (end 56 59.7) (width 0.2) (layer "B.Cu") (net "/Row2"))
 (segment (start 60.112 79.052) (end 62.06 81) (width 0.2) (layer "B.Cu") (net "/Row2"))
 (segment (start 58.75 77.69) (end 60.112 79.052) (width 0.2) (layer "B.Cu") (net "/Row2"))
 (segment (start 80 81) (end 96.518 81) (width 0.2) (layer "B.Cu") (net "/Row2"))
 (segment (start 80.94 44) (end 82.94 42) (width 0.2) (layer "B.Cu") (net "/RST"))
 (segment (start 101.9 43.834315) (end 101.9 45.9) (width 0.2) (layer "B.Cu") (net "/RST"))
 (segment (start 102.75 46.75) (end 107.75 46.75) (width 0.2) (layer "B.Cu") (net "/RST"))
 (segment (start 100.065685 42) (end 101.9 43.834315) (width 0.2) (layer "B.Cu") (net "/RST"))
 (segment (start 82.94 42) (end 100.065685 42) (width 0.2) (layer "B.Cu") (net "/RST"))
 (segment (start 101.9 45.9) (end 102.75 46.75) (width 0.2) (layer "B.Cu") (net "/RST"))
 (segment (start 107.75 46.75) (end 114.25 46.75) (width 0.2) (layer "B.Cu") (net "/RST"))
 (segment (start 101.5 49.75) (end 101.5 44) (width 0.2) (layer "B.Cu") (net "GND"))
 (segment (start 78.4 59.24) (end 78.4 57.6) (width 0.2) (layer "B.Cu") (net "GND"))
 (segment (start 84.98 42.5) (end 83.48 44) (width 0.2) (layer "B.Cu") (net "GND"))
 (segment (start 83.48 52.52) (end 83.48 44) (width 0.2) (layer "B.Cu") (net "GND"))
 (segment (start 78.4 57.6) (end 83.48 52.52) (width 0.2) (layer "B.Cu") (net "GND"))
 (segment (start 107.5 51.5) (end 107.75 51.25) (width 0.2) (layer "B.Cu") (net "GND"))
 (segment (start 100 42.5) (end 84.98 42.5) (width 0.2) (layer "B.Cu") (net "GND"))
 (segment (start 103 51.25) (end 101.5 49.75) (width 0.2) (layer "B.Cu") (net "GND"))
 (segment (start 107.75 51.25) (end 103 51.25) (width 0.2) (layer "B.Cu") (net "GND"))
 (segment (start 101.5 44) (end 100 42.5) (width 0.2) (layer "B.Cu") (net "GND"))
 (segment (start 107.75 51.25) (end 114.25 51.25) (width 0.2) (layer "B.Cu") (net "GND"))
 (segment (start 70.78 59.24) (end 70.78 58.28) (width 0.2) (layer "B.Cu") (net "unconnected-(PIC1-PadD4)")))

